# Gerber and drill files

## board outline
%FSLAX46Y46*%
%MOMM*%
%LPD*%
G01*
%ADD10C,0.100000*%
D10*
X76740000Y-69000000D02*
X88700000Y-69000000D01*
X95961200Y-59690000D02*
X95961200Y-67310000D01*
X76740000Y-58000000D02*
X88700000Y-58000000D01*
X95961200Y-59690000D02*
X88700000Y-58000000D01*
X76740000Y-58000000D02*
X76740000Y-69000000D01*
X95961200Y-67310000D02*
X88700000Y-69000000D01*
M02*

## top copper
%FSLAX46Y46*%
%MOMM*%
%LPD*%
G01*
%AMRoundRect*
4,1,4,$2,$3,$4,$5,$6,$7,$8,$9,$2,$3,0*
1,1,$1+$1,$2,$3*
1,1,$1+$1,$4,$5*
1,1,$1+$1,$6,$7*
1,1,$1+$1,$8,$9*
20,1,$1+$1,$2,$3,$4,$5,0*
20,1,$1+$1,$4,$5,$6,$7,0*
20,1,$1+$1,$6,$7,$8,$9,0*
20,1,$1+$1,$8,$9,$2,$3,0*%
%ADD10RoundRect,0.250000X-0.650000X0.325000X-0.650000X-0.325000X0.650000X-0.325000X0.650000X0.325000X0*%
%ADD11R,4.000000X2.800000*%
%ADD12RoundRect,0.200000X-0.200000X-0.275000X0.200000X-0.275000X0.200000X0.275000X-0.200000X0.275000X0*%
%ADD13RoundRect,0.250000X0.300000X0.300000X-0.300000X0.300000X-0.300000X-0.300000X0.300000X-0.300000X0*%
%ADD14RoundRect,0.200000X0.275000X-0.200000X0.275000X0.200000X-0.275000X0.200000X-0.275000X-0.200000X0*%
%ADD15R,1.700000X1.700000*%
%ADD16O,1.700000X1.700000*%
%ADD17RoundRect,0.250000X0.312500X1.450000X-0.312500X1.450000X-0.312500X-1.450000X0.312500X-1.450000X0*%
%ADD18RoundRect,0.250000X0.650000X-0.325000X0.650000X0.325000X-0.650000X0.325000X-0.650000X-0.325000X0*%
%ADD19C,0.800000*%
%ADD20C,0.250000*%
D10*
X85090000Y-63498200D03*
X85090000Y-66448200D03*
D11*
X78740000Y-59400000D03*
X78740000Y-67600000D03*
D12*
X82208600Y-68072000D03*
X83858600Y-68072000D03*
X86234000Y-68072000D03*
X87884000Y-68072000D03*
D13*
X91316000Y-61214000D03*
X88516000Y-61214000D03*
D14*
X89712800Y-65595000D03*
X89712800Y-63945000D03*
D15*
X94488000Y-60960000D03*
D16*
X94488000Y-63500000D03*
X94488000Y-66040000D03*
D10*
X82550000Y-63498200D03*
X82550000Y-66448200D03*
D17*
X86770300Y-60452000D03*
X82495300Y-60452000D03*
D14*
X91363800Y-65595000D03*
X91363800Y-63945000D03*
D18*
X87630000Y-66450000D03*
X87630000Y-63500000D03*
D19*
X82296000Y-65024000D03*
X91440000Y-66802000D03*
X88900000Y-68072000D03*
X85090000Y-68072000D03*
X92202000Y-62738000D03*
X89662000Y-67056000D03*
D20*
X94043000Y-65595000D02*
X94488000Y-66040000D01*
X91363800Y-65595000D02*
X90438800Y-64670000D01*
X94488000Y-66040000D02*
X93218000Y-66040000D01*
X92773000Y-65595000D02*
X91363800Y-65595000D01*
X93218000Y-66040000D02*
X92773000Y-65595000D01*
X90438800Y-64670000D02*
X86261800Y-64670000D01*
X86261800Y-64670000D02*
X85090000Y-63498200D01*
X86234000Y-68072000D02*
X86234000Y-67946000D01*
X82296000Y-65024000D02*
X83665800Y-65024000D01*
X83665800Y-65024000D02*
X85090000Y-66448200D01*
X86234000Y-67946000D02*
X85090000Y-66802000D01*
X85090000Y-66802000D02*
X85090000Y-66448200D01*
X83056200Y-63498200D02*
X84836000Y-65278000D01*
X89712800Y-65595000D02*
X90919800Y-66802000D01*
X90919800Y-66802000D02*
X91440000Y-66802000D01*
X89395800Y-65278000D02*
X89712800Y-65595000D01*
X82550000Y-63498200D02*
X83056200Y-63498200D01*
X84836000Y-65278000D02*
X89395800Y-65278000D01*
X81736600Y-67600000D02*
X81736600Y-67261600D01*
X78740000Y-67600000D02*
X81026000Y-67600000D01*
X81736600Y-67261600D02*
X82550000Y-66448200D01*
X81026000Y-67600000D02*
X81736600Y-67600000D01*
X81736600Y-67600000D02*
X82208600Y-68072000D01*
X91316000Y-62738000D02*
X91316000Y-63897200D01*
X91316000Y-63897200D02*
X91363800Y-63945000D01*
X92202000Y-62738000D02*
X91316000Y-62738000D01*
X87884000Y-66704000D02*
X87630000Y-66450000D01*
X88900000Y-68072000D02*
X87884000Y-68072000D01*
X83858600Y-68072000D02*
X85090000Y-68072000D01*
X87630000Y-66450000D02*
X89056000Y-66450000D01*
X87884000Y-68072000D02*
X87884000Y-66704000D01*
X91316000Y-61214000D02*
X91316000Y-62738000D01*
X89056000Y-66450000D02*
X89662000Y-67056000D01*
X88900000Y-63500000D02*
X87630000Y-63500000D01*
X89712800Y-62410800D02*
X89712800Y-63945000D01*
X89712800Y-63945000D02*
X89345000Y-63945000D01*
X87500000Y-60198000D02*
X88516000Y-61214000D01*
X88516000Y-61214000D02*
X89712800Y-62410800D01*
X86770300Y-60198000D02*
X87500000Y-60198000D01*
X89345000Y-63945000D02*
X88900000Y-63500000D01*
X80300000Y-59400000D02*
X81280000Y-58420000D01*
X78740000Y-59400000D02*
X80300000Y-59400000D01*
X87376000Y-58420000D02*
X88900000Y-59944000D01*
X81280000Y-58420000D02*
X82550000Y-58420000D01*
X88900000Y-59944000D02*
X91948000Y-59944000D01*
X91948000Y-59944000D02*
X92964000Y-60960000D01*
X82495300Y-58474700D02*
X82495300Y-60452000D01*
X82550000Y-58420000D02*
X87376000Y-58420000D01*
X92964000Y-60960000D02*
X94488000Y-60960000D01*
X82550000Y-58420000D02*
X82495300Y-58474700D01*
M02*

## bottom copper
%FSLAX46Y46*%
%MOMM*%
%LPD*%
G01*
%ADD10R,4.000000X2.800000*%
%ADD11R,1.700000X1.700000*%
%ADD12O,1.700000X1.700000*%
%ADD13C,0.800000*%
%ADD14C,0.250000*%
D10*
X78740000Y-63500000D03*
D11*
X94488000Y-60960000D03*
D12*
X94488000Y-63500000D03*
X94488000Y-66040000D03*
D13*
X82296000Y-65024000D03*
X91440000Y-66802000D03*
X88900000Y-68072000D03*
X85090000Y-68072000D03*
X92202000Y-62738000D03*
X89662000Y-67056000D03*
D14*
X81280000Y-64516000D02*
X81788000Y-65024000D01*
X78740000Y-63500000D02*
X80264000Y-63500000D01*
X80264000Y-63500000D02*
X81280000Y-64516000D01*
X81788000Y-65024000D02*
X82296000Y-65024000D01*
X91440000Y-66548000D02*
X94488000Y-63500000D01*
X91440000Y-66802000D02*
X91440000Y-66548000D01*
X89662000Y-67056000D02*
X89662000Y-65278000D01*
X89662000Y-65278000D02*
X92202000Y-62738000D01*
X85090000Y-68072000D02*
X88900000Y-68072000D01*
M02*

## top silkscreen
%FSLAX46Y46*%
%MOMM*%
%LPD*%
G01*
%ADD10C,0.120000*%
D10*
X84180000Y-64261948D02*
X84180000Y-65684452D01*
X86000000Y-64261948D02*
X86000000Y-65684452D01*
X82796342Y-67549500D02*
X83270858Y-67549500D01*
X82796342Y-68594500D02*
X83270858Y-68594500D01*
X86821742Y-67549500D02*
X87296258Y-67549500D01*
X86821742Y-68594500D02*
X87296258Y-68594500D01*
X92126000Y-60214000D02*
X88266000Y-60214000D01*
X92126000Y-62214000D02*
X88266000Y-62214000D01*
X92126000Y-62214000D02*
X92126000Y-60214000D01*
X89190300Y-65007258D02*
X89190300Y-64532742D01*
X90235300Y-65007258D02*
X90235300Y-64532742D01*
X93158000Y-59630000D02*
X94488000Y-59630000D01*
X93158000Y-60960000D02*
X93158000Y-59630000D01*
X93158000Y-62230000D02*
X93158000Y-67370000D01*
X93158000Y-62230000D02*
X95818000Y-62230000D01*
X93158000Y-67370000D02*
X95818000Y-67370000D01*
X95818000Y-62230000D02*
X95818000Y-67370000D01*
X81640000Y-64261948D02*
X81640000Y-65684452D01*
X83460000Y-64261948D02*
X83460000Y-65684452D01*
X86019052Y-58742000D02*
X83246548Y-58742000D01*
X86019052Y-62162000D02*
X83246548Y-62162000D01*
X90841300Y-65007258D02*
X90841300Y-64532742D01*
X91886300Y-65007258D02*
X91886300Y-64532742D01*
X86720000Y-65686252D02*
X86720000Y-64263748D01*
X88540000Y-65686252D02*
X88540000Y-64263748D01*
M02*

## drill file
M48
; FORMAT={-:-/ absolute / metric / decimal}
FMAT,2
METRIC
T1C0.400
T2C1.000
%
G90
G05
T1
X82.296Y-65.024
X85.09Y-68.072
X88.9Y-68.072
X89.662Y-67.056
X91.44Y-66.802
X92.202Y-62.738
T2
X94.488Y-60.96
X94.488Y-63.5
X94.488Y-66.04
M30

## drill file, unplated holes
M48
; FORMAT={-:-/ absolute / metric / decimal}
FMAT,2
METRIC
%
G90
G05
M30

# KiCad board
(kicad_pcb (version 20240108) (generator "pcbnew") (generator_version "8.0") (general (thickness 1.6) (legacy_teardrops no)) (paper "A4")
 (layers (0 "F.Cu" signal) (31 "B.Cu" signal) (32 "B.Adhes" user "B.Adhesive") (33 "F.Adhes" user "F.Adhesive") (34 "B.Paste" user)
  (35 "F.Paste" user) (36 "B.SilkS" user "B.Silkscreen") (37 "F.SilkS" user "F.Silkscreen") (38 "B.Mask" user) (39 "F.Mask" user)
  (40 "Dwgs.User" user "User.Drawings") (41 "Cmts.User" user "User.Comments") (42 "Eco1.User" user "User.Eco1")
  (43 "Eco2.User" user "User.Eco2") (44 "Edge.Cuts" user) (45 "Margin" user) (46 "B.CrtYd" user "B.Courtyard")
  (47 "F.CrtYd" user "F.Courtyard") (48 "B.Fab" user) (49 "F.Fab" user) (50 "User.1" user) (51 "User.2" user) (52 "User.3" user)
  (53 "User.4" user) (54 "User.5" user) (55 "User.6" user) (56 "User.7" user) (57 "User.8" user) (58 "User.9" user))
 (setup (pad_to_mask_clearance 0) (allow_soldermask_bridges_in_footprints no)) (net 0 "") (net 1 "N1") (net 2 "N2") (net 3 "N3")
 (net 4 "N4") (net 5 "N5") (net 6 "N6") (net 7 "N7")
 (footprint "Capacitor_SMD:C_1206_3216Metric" (layer "F.Cu") (at 85.09 64.9732 -90)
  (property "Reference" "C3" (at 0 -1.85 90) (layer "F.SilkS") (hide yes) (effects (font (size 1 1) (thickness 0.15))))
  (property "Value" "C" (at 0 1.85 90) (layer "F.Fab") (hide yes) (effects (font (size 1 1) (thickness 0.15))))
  (fp_line (start -0.711252 0.91) (end 0.711252 0.91) (stroke (width 0.12) (type solid)) (layer "F.SilkS"))
  (fp_line (start -0.711252 -0.91) (end 0.711252 -0.91) (stroke (width 0.12) (type solid)) (layer "F.SilkS"))
  (pad "1" smd roundrect (at -1.475 0 270) (size 1.15 1.8) (layers "F.Cu" "F.Paste" "F.Mask") (roundrect_rratio 0.2173913043) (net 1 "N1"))
  (pad "2" smd roundrect (at 1.475 0 270) (size 1.15 1.8) (layers "F.Cu" "F.Paste" "F.Mask") (roundrect_rratio 0.2173913043) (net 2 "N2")))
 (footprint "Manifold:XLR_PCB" (layer "F.Cu") (at 78.74 63.5)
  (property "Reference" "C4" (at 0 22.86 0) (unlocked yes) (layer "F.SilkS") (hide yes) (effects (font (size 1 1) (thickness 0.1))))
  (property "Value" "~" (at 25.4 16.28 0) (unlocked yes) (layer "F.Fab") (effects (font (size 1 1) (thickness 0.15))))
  (pad "1" connect rect (at 0 -4.1) (size 4 2.8) (layers "F.Cu" "F.Mask") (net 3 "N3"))
  (pad "2" connect rect (at 0 4.1) (size 4 2.8) (layers "F.Cu" "F.Mask") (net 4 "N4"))
  (pad "3" connect rect (at 0 0) (size 4 2.8) (layers "B.Cu" "B.Mask") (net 2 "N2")))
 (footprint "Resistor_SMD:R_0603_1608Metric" (layer "F.Cu") (at 83.0336 68.072)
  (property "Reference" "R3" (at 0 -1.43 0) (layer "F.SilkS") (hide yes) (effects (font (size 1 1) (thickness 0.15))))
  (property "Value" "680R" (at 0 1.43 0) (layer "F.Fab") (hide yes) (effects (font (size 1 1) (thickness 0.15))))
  (fp_line (start -0.237258 -0.5225) (end 0.237258 -0.5225) (stroke (width 0.12) (type solid)) (layer "F.SilkS"))
  (fp_line (start -0.237258 0.5225) (end 0.237258 0.5225) (stroke (width 0.12) (type solid)) (layer "F.SilkS"))
  (pad "1" smd roundrect (at -0.825 0) (size 0.8 0.95) (layers "F.Cu" "F.Paste" "F.Mask") (roundrect_rratio 0.25) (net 4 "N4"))
  (pad "2" smd roundrect (at 0.825 0) (size 0.8 0.95) (layers "F.Cu" "F.Paste" "F.Mask") (roundrect_rratio 0.25) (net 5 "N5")))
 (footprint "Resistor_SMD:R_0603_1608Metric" (layer "F.Cu") (at 87.059 68.072)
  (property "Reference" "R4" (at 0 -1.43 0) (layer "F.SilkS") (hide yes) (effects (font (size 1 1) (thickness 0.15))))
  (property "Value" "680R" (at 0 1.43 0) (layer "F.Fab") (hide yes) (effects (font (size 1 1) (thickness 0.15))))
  (fp_line (start -0.237258 -0.5225) (end 0.237258 -0.5225) (stroke (width 0.12) (type solid)) (layer "F.SilkS"))
  (fp_line (start -0.237258 0.5225) (end 0.237258 0.5225) (stroke (width 0.12) (type solid)) (layer "F.SilkS"))
  (pad "1" smd roundrect (at -0.825 0) (size 0.8 0.95) (layers "F.Cu" "F.Paste" "F.Mask") (roundrect_rratio 0.25) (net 2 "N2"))
  (pad "2" smd roundrect (at 0.825 0) (size 0.8 0.95) (layers "F.Cu" "F.Paste" "F.Mask") (roundrect_rratio 0.25) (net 5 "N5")))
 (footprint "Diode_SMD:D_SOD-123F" (layer "F.Cu") (at 89.916 61.214 180)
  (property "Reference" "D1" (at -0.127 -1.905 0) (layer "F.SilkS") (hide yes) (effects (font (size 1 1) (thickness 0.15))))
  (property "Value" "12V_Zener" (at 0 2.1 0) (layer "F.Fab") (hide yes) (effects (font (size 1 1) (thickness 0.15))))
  (fp_line (start -2.21 1) (end 1.65 1) (stroke (width 0.12) (type solid)) (layer "F.SilkS"))
  (fp_line (start -2.21 -1) (end 1.65 -1) (stroke (width 0.12) (type solid)) (layer "F.SilkS"))
  (fp_line (start -2.21 -1) (end -2.21 1) (stroke (width 0.12) (type solid)) (layer "F.SilkS"))
  (pad "1" smd roundrect (at -1.4 0 180) (size 1.1 1.1) (layers "F.Cu" "F.Paste" "F.Mask") (roundrect_rratio 0.2272727273) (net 5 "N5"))
  (pad "2" smd roundrect (at 1.4 0 180) (size 1.1 1.1) (layers "F.Cu" "F.Paste" "F.Mask") (roundrect_rratio 0.2272727273) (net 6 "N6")))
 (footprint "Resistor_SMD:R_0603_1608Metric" (layer "F.Cu") (at 89.7128 64.77 90)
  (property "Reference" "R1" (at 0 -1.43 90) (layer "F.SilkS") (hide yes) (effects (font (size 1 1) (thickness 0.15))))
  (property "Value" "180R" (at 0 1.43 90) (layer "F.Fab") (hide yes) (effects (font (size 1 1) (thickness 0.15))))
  (fp_line (start -0.237258 -0.5225) (end 0.237258 -0.5225) (stroke (width 0.12) (type solid)) (layer "F.SilkS"))
  (fp_line (start -0.237258 0.5225) (end 0.237258 0.5225) (stroke (width 0.12) (type solid)) (layer "F.SilkS"))
  (pad "1" smd roundrect (at -0.825 0 90) (size 0.8 0.95) (layers "F.Cu" "F.Paste" "F.Mask") (roundrect_rratio 0.25) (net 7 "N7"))
  (pad "2" smd roundrect (at 0.825 0 90) (size 0.8 0.95) (layers "F.Cu" "F.Paste" "F.Mask") (roundrect_rratio 0.25) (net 6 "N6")))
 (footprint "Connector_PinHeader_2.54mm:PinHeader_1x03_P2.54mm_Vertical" (layer "F.Cu") (at 94.488 60.96)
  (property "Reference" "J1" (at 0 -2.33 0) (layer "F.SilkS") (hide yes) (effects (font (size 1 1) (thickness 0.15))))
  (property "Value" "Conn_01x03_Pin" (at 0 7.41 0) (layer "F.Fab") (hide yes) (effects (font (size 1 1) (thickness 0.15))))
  (fp_line (start -1.33 -1.33) (end 0 -1.33) (stroke (width 0.12) (type solid)) (layer "F.SilkS"))
  (fp_line (start -1.33 0) (end -1.33 -1.33) (stroke (width 0.12) (type solid)) (layer "F.SilkS"))
  (fp_line (start -1.33 1.27) (end -1.33 6.41) (stroke (width 0.12) (type solid)) (layer "F.SilkS"))
  (fp_line (start -1.33 1.27) (end 1.33 1.27) (stroke (width 0.12) (type solid)) (layer "F.SilkS"))
  (fp_line (start -1.33 6.41) (end 1.33 6.41) (stroke (width 0.12) (type solid)) (layer "F.SilkS"))
  (fp_line (start 1.33 1.27) (end 1.33 6.41) (stroke (width 0.12) (type solid)) (layer "F.SilkS"))
  (pad "1" thru_hole rect (at 0 0) (size 1.7 1.7) (drill 1) (layers "*.Cu" "*.Mask") (remove_unused_layers no) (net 3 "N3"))
  (pad "2" thru_hole oval (at 0 2.54) (size 1.7 1.7) (drill 1) (layers "*.Cu" "*.Mask") (remove_unused_layers no) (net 7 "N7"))
  (pad "3" thru_hole oval (at 0 5.08) (size 1.7 1.7) (drill 1) (layers "*.Cu" "*.Mask") (remove_unused_layers no) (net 1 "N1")))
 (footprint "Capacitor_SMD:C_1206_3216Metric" (layer "F.Cu") (at 82.55 64.9732 -90)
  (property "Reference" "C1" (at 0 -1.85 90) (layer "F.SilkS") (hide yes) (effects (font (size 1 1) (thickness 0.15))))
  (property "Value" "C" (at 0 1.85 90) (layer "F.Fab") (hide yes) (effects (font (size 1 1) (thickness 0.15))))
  (fp_line (start -0.711252 0.91) (end 0.711252 0.91) (stroke (width 0.12) (type solid)) (layer "F.SilkS"))
  (fp_line (start -0.711252 -0.91) (end 0.711252 -0.91) (stroke (width 0.12) (type solid)) (layer "F.SilkS"))
  (pad "1" smd roundrect (at -1.475 0 270) (size 1.15 1.8) (layers "F.Cu" "F.Paste" "F.Mask") (roundrect_rratio 0.2173913043) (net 7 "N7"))
  (pad "2" smd roundrect (at 1.475 0 270) (size 1.15 1.8) (layers "F.Cu" "F.Paste" "F.Mask") (roundrect_rratio 0.2173913043) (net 4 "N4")))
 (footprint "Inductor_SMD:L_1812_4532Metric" (layer "F.Cu") (at 84.6328 60.452 180)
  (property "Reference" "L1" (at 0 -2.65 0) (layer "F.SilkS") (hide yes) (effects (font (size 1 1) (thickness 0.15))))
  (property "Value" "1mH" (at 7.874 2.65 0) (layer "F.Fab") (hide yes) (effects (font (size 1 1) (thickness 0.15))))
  (fp_line (start -1.386252 1.71) (end 1.386252 1.71) (stroke (width 0.12) (type solid)) (layer "F.SilkS"))
  (fp_line (start -1.386252 -1.71) (end 1.386252 -1.71) (stroke (width 0.12) (type solid)) (layer "F.SilkS"))
  (pad "1" smd roundrect (at -2.1375 0 180) (size 1.125 3.4) (layers "F.Cu" "F.Paste" "F.Mask") (roundrect_rratio 0.2222222222) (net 6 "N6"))
  (pad "2" smd roundrect (at 2.1375 0 180) (size 1.125 3.4) (layers "F.Cu" "F.Paste" "F.Mask") (roundrect_rratio 0.2222222222) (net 3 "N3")))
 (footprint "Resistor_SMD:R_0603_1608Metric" (layer "F.Cu") (at 91.3638 64.77 90)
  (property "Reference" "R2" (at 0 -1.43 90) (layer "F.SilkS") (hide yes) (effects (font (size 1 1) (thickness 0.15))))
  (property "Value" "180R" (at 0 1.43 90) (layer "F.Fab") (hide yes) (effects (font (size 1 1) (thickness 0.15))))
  (fp_line (start -0.237258 -0.5225) (end 0.237258 -0.5225) (stroke (width 0.12) (type solid)) (layer "F.SilkS"))
  (fp_line (start -0.237258 0.5225) (end 0.237258 0.5225) (stroke (width 0.12) (type solid)) (layer "F.SilkS"))
  (pad "1" smd roundrect (at -0.825 0 90) (size 0.8 0.95) (layers "F.Cu" "F.Paste" "F.Mask") (roundrect_rratio 0.25) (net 1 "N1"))
  (pad "2" smd roundrect (at 0.825 0 90) (size 0.8 0.95) (layers "F.Cu" "F.Paste" "F.Mask") (roundrect_rratio 0.25) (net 5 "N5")))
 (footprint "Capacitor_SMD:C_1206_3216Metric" (layer "F.Cu") (at 87.63 64.975 90)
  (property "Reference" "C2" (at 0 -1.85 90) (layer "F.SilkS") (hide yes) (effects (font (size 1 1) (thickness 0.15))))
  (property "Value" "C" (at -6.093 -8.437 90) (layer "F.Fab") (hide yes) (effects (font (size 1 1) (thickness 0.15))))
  (fp_line (start -0.711252 -0.91) (end 0.711252 -0.91) (stroke (width 0.12) (type solid)) (layer "F.SilkS"))
  (fp_line (start -0.711252 0.91) (end 0.711252 0.91) (stroke (width 0.12) (type solid)) (layer "F.SilkS"))
  (pad "1" smd roundrect (at -1.475 0 90) (size 1.15 1.8) (layers "F.Cu" "F.Paste" "F.Mask") (roundrect_rratio 0.2173913043) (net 5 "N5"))
  (pad "2" smd roundrect (at 1.475 0 90) (size 1.15 1.8) (layers "F.Cu" "F.Paste" "F.Mask") (roundrect_rratio 0.2173913043) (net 6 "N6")))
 (gr_line (start 76.74 69) (end 88.7 69) (stroke (width 0.1) (type default)) (layer "Edge.Cuts"))
 (gr_line (start 95.9612 59.69) (end 95.9612 67.31) (stroke (width 0.1) (type default)) (layer "Edge.Cuts"))
 (gr_line (start 76.74 58) (end 88.7 58) (stroke (width 0.1) (type default)) (layer "Edge.Cuts"))
 (gr_line (start 95.9612 59.69) (end 88.7 58) (stroke (width 0.1) (type default)) (layer "Edge.Cuts"))
 (gr_line (start 76.74 58) (end 76.74 69) (stroke (width 0.1) (type default)) (layer "Edge.Cuts"))
 (gr_line (start 95.9612 67.31) (end 88.7 69) (stroke (width 0.1) (type default)) (layer "Edge.Cuts"))
 (segment (start 94.043 65.595) (end 94.488 66.04) (width 0.25) (layer "F.Cu") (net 1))
 (segment (start 91.3638 65.595) (end 90.4388 64.67) (width 0.25) (layer "F.Cu") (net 1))
 (segment (start 94.488 66.04) (end 93.218 66.04) (width 0.25) (layer "F.Cu") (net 1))
 (segment (start 92.773 65.595) (end 91.3638 65.595) (width 0.25) (layer "F.Cu") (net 1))
 (segment (start 93.218 66.04) (end 92.773 65.595) (width 0.25) (layer "F.Cu") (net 1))
 (segment (start 90.4388 64.67) (end 86.2618 64.67) (width 0.25) (layer "F.Cu") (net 1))
 (segment (start 86.2618 64.67) (end 85.09 63.4982) (width 0.25) (layer "F.Cu") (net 1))
 (segment (start 86.234 68.072) (end 86.234 67.946) (width 0.25) (layer "F.Cu") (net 2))
 (segment (start 82.296 65.024) (end 83.6658 65.024) (width 0.25) (layer "F.Cu") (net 2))
 (segment (start 83.6658 65.024) (end 85.09 66.4482) (width 0.25) (layer "F.Cu") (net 2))
 (segment (start 86.234 67.946) (end 85.09 66.802) (width 0.25) (layer "F.Cu") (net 2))
 (segment (start 85.09 66.802) (end 85.09 66.4482) (width 0.25) (layer "F.Cu") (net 2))
 (via (at 82.296 65.024) (size 0.8) (drill 0.4) (layers "F.Cu" "B.Cu") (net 2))
 (segment (start 81.28 64.516) (end 81.788 65.024) (width 0.25) (layer "B.Cu") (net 2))
 (segment (start 78.74 63.5) (end 80.264 63.5) (width 0.25) (layer "B.Cu") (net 2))
 (segment (start 80.264 63.5) (end 81.28 64.516) (width 0.25) (layer "B.Cu") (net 2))
 (segment (start 81.788 65.024) (end 82.296 65.024) (width 0.25) (layer "B.Cu") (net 2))
 (segment (start 83.0562 63.4982) (end 84.836 65.278) (width 0.25) (layer "F.Cu") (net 7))
 (segment (start 89.7128 65.595) (end 90.9198 66.802) (width 0.25) (layer "F.Cu") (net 7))
 (segment (start 90.9198 66.802) (end 91.44 66.802) (width 0.25) (layer "F.Cu") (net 7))
 (segment (start 89.3958 65.278) (end 89.7128 65.595) (width 0.25) (layer "F.Cu") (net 7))
 (segment (start 82.55 63.4982) (end 83.0562 63.4982) (width 0.25) (layer "F.Cu") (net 7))
 (segment (start 84.836 65.278) (end 89.3958 65.278) (width 0.25) (layer "F.Cu") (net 7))
 (via (at 91.44 66.802) (size 0.8) (drill 0.4) (layers "F.Cu" "B.Cu") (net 7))
 (segment (start 91.44 66.548) (end 94.488 63.5) (width 0.25) (layer "B.Cu") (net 7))
 (segment (start 91.44 66.802) (end 91.44 66.548) (width 0.25) (layer "B.Cu") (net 7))
 (segment (start 81.7366 67.6) (end 81.7366 67.2616) (width 0.25) (layer "F.Cu") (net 4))
 (segment (start 78.74 67.6) (end 81.026 67.6) (width 0.25) (layer "F.Cu") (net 4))
 (segment (start 81.7366 67.2616) (end 82.55 66.4482) (width 0.25) (layer "F.Cu") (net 4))
 (segment (start 81.026 67.6) (end 81.7366 67.6) (width 0.25) (layer "F.Cu") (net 4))
 (segment (start 81.7366 67.6) (end 82.2086 68.072) (width 0.25) (layer "F.Cu") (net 4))
 (segment (start 91.316 62.738) (end 91.316 63.8972) (width 0.25) (layer "F.Cu") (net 5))
 (segment (start 91.316 63.8972) (end 91.3638 63.945) (width 0.25) (layer "F.Cu") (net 5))
 (segment (start 92.202 62.738) (end 91.316 62.738) (width 0.25) (layer "F.Cu") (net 5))
 (segment (start 87.884 66.704) (end 87.63 66.45) (width 0.25) (layer "F.Cu") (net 5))
 (segment (start 88.9 68.072) (end 87.884 68.072) (width 0.25) (layer "F.Cu") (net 5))
 (segment (start 83.8586 68.072) (end 85.09 68.072) (width 0.25) (layer "F.Cu") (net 5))
 (segment (start 87.63 66.45) (end 89.056 66.45) (width 0.25) (layer "F.Cu") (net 5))
 (segment (start 87.884 68.072) (end 87.884 66.704) (width 0.25) (layer "F.Cu") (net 5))
 (segment (start 91.316 61.214) (end 91.316 62.738) (width 0.25) (layer "F.Cu") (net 5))
 (segment (start 89.056 66.45) (end 89.662 67.056) (width 0.25) (layer "F.Cu") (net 5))
 (via (at 88.9 68.072) (size 0.8) (drill 0.4) (layers "F.Cu" "B.Cu") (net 5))
 (via (at 85.09 68.072) (size 0.8) (drill 0.4) (layers "F.Cu" "B.Cu") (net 5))
 (via (at 92.202 62.738) (size 0.8) (drill 0.4) (layers "F.Cu" "B.Cu") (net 5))
 (via (at 89.662 67.056) (size 0.8) (drill 0.4) (layers "F.Cu" "B.Cu") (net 5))
 (segment (start 89.662 67.056) (end 89.662 65.278) (width 0.25) (layer "B.Cu") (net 5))
 (segment (start 89.662 65.278) (end 92.202 62.738) (width 0.25) (layer "B.Cu") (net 5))
 (segment (start 85.09 68.072) (end 88.9 68.072) (width 0.25) (layer "B.Cu") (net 5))
 (segment (start 88.9 63.5) (end 87.63 63.5) (width 0.25) (layer "F.Cu") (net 6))
 (segment (start 89.7128 62.4108) (end 89.7128 63.945) (width 0.25) (layer "F.Cu") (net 6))
 (segment (start 89.7128 63.945) (end 89.345 63.945) (width 0.25) (layer "F.Cu") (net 6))
 (segment (start 87.5 60.198) (end 88.516 61.214) (width 0.25) (layer "F.Cu") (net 6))
 (segment (start 88.516 61.214) (end 89.7128 62.4108) (width 0.25) (layer "F.Cu") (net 6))
 (segment (start 86.7703 60.198) (end 87.5 60.198) (width 0.25) (layer "F.Cu") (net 6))
 (segment (start 89.345 63.945) (end 88.9 63.5) (width 0.25) (layer "F.Cu") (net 6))
 (segment (start 80.3 59.4) (end 81.28 58.42) (width 0.25) (layer "F.Cu") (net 3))
 (segment (start 78.74 59.4) (end 80.3 59.4) (width 0.25) (layer "F.Cu") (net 3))
 (segment (start 87.376 58.42) (end 88.9 59.944) (width 0.25) (layer "F.Cu") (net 3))
 (segment (start 81.28 58.42) (end 82.55 58.42) (width 0.25) (layer "F.Cu") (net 3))
 (segment (start 88.9 59.944) (end 91.948 59.944) (width 0.25) (layer "F.Cu") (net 3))
 (segment (start 91.948 59.944) (end 92.964 60.96) (width 0.25) (layer "F.Cu") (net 3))
 (segment (start 82.4953 58.4747) (end 82.4953 60.452) (width 0.25) (layer "F.Cu") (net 3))
 (segment (start 82.55 58.42) (end 87.376 58.42) (width 0.25) (layer "F.Cu") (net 3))
 (segment (start 92.964 60.96) (end 94.488 60.96) (width 0.25) (layer "F.Cu") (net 3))
 (segment (start 82.55 58.42) (end 82.4953 58.4747) (width 0.25) (layer "F.Cu") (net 3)))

